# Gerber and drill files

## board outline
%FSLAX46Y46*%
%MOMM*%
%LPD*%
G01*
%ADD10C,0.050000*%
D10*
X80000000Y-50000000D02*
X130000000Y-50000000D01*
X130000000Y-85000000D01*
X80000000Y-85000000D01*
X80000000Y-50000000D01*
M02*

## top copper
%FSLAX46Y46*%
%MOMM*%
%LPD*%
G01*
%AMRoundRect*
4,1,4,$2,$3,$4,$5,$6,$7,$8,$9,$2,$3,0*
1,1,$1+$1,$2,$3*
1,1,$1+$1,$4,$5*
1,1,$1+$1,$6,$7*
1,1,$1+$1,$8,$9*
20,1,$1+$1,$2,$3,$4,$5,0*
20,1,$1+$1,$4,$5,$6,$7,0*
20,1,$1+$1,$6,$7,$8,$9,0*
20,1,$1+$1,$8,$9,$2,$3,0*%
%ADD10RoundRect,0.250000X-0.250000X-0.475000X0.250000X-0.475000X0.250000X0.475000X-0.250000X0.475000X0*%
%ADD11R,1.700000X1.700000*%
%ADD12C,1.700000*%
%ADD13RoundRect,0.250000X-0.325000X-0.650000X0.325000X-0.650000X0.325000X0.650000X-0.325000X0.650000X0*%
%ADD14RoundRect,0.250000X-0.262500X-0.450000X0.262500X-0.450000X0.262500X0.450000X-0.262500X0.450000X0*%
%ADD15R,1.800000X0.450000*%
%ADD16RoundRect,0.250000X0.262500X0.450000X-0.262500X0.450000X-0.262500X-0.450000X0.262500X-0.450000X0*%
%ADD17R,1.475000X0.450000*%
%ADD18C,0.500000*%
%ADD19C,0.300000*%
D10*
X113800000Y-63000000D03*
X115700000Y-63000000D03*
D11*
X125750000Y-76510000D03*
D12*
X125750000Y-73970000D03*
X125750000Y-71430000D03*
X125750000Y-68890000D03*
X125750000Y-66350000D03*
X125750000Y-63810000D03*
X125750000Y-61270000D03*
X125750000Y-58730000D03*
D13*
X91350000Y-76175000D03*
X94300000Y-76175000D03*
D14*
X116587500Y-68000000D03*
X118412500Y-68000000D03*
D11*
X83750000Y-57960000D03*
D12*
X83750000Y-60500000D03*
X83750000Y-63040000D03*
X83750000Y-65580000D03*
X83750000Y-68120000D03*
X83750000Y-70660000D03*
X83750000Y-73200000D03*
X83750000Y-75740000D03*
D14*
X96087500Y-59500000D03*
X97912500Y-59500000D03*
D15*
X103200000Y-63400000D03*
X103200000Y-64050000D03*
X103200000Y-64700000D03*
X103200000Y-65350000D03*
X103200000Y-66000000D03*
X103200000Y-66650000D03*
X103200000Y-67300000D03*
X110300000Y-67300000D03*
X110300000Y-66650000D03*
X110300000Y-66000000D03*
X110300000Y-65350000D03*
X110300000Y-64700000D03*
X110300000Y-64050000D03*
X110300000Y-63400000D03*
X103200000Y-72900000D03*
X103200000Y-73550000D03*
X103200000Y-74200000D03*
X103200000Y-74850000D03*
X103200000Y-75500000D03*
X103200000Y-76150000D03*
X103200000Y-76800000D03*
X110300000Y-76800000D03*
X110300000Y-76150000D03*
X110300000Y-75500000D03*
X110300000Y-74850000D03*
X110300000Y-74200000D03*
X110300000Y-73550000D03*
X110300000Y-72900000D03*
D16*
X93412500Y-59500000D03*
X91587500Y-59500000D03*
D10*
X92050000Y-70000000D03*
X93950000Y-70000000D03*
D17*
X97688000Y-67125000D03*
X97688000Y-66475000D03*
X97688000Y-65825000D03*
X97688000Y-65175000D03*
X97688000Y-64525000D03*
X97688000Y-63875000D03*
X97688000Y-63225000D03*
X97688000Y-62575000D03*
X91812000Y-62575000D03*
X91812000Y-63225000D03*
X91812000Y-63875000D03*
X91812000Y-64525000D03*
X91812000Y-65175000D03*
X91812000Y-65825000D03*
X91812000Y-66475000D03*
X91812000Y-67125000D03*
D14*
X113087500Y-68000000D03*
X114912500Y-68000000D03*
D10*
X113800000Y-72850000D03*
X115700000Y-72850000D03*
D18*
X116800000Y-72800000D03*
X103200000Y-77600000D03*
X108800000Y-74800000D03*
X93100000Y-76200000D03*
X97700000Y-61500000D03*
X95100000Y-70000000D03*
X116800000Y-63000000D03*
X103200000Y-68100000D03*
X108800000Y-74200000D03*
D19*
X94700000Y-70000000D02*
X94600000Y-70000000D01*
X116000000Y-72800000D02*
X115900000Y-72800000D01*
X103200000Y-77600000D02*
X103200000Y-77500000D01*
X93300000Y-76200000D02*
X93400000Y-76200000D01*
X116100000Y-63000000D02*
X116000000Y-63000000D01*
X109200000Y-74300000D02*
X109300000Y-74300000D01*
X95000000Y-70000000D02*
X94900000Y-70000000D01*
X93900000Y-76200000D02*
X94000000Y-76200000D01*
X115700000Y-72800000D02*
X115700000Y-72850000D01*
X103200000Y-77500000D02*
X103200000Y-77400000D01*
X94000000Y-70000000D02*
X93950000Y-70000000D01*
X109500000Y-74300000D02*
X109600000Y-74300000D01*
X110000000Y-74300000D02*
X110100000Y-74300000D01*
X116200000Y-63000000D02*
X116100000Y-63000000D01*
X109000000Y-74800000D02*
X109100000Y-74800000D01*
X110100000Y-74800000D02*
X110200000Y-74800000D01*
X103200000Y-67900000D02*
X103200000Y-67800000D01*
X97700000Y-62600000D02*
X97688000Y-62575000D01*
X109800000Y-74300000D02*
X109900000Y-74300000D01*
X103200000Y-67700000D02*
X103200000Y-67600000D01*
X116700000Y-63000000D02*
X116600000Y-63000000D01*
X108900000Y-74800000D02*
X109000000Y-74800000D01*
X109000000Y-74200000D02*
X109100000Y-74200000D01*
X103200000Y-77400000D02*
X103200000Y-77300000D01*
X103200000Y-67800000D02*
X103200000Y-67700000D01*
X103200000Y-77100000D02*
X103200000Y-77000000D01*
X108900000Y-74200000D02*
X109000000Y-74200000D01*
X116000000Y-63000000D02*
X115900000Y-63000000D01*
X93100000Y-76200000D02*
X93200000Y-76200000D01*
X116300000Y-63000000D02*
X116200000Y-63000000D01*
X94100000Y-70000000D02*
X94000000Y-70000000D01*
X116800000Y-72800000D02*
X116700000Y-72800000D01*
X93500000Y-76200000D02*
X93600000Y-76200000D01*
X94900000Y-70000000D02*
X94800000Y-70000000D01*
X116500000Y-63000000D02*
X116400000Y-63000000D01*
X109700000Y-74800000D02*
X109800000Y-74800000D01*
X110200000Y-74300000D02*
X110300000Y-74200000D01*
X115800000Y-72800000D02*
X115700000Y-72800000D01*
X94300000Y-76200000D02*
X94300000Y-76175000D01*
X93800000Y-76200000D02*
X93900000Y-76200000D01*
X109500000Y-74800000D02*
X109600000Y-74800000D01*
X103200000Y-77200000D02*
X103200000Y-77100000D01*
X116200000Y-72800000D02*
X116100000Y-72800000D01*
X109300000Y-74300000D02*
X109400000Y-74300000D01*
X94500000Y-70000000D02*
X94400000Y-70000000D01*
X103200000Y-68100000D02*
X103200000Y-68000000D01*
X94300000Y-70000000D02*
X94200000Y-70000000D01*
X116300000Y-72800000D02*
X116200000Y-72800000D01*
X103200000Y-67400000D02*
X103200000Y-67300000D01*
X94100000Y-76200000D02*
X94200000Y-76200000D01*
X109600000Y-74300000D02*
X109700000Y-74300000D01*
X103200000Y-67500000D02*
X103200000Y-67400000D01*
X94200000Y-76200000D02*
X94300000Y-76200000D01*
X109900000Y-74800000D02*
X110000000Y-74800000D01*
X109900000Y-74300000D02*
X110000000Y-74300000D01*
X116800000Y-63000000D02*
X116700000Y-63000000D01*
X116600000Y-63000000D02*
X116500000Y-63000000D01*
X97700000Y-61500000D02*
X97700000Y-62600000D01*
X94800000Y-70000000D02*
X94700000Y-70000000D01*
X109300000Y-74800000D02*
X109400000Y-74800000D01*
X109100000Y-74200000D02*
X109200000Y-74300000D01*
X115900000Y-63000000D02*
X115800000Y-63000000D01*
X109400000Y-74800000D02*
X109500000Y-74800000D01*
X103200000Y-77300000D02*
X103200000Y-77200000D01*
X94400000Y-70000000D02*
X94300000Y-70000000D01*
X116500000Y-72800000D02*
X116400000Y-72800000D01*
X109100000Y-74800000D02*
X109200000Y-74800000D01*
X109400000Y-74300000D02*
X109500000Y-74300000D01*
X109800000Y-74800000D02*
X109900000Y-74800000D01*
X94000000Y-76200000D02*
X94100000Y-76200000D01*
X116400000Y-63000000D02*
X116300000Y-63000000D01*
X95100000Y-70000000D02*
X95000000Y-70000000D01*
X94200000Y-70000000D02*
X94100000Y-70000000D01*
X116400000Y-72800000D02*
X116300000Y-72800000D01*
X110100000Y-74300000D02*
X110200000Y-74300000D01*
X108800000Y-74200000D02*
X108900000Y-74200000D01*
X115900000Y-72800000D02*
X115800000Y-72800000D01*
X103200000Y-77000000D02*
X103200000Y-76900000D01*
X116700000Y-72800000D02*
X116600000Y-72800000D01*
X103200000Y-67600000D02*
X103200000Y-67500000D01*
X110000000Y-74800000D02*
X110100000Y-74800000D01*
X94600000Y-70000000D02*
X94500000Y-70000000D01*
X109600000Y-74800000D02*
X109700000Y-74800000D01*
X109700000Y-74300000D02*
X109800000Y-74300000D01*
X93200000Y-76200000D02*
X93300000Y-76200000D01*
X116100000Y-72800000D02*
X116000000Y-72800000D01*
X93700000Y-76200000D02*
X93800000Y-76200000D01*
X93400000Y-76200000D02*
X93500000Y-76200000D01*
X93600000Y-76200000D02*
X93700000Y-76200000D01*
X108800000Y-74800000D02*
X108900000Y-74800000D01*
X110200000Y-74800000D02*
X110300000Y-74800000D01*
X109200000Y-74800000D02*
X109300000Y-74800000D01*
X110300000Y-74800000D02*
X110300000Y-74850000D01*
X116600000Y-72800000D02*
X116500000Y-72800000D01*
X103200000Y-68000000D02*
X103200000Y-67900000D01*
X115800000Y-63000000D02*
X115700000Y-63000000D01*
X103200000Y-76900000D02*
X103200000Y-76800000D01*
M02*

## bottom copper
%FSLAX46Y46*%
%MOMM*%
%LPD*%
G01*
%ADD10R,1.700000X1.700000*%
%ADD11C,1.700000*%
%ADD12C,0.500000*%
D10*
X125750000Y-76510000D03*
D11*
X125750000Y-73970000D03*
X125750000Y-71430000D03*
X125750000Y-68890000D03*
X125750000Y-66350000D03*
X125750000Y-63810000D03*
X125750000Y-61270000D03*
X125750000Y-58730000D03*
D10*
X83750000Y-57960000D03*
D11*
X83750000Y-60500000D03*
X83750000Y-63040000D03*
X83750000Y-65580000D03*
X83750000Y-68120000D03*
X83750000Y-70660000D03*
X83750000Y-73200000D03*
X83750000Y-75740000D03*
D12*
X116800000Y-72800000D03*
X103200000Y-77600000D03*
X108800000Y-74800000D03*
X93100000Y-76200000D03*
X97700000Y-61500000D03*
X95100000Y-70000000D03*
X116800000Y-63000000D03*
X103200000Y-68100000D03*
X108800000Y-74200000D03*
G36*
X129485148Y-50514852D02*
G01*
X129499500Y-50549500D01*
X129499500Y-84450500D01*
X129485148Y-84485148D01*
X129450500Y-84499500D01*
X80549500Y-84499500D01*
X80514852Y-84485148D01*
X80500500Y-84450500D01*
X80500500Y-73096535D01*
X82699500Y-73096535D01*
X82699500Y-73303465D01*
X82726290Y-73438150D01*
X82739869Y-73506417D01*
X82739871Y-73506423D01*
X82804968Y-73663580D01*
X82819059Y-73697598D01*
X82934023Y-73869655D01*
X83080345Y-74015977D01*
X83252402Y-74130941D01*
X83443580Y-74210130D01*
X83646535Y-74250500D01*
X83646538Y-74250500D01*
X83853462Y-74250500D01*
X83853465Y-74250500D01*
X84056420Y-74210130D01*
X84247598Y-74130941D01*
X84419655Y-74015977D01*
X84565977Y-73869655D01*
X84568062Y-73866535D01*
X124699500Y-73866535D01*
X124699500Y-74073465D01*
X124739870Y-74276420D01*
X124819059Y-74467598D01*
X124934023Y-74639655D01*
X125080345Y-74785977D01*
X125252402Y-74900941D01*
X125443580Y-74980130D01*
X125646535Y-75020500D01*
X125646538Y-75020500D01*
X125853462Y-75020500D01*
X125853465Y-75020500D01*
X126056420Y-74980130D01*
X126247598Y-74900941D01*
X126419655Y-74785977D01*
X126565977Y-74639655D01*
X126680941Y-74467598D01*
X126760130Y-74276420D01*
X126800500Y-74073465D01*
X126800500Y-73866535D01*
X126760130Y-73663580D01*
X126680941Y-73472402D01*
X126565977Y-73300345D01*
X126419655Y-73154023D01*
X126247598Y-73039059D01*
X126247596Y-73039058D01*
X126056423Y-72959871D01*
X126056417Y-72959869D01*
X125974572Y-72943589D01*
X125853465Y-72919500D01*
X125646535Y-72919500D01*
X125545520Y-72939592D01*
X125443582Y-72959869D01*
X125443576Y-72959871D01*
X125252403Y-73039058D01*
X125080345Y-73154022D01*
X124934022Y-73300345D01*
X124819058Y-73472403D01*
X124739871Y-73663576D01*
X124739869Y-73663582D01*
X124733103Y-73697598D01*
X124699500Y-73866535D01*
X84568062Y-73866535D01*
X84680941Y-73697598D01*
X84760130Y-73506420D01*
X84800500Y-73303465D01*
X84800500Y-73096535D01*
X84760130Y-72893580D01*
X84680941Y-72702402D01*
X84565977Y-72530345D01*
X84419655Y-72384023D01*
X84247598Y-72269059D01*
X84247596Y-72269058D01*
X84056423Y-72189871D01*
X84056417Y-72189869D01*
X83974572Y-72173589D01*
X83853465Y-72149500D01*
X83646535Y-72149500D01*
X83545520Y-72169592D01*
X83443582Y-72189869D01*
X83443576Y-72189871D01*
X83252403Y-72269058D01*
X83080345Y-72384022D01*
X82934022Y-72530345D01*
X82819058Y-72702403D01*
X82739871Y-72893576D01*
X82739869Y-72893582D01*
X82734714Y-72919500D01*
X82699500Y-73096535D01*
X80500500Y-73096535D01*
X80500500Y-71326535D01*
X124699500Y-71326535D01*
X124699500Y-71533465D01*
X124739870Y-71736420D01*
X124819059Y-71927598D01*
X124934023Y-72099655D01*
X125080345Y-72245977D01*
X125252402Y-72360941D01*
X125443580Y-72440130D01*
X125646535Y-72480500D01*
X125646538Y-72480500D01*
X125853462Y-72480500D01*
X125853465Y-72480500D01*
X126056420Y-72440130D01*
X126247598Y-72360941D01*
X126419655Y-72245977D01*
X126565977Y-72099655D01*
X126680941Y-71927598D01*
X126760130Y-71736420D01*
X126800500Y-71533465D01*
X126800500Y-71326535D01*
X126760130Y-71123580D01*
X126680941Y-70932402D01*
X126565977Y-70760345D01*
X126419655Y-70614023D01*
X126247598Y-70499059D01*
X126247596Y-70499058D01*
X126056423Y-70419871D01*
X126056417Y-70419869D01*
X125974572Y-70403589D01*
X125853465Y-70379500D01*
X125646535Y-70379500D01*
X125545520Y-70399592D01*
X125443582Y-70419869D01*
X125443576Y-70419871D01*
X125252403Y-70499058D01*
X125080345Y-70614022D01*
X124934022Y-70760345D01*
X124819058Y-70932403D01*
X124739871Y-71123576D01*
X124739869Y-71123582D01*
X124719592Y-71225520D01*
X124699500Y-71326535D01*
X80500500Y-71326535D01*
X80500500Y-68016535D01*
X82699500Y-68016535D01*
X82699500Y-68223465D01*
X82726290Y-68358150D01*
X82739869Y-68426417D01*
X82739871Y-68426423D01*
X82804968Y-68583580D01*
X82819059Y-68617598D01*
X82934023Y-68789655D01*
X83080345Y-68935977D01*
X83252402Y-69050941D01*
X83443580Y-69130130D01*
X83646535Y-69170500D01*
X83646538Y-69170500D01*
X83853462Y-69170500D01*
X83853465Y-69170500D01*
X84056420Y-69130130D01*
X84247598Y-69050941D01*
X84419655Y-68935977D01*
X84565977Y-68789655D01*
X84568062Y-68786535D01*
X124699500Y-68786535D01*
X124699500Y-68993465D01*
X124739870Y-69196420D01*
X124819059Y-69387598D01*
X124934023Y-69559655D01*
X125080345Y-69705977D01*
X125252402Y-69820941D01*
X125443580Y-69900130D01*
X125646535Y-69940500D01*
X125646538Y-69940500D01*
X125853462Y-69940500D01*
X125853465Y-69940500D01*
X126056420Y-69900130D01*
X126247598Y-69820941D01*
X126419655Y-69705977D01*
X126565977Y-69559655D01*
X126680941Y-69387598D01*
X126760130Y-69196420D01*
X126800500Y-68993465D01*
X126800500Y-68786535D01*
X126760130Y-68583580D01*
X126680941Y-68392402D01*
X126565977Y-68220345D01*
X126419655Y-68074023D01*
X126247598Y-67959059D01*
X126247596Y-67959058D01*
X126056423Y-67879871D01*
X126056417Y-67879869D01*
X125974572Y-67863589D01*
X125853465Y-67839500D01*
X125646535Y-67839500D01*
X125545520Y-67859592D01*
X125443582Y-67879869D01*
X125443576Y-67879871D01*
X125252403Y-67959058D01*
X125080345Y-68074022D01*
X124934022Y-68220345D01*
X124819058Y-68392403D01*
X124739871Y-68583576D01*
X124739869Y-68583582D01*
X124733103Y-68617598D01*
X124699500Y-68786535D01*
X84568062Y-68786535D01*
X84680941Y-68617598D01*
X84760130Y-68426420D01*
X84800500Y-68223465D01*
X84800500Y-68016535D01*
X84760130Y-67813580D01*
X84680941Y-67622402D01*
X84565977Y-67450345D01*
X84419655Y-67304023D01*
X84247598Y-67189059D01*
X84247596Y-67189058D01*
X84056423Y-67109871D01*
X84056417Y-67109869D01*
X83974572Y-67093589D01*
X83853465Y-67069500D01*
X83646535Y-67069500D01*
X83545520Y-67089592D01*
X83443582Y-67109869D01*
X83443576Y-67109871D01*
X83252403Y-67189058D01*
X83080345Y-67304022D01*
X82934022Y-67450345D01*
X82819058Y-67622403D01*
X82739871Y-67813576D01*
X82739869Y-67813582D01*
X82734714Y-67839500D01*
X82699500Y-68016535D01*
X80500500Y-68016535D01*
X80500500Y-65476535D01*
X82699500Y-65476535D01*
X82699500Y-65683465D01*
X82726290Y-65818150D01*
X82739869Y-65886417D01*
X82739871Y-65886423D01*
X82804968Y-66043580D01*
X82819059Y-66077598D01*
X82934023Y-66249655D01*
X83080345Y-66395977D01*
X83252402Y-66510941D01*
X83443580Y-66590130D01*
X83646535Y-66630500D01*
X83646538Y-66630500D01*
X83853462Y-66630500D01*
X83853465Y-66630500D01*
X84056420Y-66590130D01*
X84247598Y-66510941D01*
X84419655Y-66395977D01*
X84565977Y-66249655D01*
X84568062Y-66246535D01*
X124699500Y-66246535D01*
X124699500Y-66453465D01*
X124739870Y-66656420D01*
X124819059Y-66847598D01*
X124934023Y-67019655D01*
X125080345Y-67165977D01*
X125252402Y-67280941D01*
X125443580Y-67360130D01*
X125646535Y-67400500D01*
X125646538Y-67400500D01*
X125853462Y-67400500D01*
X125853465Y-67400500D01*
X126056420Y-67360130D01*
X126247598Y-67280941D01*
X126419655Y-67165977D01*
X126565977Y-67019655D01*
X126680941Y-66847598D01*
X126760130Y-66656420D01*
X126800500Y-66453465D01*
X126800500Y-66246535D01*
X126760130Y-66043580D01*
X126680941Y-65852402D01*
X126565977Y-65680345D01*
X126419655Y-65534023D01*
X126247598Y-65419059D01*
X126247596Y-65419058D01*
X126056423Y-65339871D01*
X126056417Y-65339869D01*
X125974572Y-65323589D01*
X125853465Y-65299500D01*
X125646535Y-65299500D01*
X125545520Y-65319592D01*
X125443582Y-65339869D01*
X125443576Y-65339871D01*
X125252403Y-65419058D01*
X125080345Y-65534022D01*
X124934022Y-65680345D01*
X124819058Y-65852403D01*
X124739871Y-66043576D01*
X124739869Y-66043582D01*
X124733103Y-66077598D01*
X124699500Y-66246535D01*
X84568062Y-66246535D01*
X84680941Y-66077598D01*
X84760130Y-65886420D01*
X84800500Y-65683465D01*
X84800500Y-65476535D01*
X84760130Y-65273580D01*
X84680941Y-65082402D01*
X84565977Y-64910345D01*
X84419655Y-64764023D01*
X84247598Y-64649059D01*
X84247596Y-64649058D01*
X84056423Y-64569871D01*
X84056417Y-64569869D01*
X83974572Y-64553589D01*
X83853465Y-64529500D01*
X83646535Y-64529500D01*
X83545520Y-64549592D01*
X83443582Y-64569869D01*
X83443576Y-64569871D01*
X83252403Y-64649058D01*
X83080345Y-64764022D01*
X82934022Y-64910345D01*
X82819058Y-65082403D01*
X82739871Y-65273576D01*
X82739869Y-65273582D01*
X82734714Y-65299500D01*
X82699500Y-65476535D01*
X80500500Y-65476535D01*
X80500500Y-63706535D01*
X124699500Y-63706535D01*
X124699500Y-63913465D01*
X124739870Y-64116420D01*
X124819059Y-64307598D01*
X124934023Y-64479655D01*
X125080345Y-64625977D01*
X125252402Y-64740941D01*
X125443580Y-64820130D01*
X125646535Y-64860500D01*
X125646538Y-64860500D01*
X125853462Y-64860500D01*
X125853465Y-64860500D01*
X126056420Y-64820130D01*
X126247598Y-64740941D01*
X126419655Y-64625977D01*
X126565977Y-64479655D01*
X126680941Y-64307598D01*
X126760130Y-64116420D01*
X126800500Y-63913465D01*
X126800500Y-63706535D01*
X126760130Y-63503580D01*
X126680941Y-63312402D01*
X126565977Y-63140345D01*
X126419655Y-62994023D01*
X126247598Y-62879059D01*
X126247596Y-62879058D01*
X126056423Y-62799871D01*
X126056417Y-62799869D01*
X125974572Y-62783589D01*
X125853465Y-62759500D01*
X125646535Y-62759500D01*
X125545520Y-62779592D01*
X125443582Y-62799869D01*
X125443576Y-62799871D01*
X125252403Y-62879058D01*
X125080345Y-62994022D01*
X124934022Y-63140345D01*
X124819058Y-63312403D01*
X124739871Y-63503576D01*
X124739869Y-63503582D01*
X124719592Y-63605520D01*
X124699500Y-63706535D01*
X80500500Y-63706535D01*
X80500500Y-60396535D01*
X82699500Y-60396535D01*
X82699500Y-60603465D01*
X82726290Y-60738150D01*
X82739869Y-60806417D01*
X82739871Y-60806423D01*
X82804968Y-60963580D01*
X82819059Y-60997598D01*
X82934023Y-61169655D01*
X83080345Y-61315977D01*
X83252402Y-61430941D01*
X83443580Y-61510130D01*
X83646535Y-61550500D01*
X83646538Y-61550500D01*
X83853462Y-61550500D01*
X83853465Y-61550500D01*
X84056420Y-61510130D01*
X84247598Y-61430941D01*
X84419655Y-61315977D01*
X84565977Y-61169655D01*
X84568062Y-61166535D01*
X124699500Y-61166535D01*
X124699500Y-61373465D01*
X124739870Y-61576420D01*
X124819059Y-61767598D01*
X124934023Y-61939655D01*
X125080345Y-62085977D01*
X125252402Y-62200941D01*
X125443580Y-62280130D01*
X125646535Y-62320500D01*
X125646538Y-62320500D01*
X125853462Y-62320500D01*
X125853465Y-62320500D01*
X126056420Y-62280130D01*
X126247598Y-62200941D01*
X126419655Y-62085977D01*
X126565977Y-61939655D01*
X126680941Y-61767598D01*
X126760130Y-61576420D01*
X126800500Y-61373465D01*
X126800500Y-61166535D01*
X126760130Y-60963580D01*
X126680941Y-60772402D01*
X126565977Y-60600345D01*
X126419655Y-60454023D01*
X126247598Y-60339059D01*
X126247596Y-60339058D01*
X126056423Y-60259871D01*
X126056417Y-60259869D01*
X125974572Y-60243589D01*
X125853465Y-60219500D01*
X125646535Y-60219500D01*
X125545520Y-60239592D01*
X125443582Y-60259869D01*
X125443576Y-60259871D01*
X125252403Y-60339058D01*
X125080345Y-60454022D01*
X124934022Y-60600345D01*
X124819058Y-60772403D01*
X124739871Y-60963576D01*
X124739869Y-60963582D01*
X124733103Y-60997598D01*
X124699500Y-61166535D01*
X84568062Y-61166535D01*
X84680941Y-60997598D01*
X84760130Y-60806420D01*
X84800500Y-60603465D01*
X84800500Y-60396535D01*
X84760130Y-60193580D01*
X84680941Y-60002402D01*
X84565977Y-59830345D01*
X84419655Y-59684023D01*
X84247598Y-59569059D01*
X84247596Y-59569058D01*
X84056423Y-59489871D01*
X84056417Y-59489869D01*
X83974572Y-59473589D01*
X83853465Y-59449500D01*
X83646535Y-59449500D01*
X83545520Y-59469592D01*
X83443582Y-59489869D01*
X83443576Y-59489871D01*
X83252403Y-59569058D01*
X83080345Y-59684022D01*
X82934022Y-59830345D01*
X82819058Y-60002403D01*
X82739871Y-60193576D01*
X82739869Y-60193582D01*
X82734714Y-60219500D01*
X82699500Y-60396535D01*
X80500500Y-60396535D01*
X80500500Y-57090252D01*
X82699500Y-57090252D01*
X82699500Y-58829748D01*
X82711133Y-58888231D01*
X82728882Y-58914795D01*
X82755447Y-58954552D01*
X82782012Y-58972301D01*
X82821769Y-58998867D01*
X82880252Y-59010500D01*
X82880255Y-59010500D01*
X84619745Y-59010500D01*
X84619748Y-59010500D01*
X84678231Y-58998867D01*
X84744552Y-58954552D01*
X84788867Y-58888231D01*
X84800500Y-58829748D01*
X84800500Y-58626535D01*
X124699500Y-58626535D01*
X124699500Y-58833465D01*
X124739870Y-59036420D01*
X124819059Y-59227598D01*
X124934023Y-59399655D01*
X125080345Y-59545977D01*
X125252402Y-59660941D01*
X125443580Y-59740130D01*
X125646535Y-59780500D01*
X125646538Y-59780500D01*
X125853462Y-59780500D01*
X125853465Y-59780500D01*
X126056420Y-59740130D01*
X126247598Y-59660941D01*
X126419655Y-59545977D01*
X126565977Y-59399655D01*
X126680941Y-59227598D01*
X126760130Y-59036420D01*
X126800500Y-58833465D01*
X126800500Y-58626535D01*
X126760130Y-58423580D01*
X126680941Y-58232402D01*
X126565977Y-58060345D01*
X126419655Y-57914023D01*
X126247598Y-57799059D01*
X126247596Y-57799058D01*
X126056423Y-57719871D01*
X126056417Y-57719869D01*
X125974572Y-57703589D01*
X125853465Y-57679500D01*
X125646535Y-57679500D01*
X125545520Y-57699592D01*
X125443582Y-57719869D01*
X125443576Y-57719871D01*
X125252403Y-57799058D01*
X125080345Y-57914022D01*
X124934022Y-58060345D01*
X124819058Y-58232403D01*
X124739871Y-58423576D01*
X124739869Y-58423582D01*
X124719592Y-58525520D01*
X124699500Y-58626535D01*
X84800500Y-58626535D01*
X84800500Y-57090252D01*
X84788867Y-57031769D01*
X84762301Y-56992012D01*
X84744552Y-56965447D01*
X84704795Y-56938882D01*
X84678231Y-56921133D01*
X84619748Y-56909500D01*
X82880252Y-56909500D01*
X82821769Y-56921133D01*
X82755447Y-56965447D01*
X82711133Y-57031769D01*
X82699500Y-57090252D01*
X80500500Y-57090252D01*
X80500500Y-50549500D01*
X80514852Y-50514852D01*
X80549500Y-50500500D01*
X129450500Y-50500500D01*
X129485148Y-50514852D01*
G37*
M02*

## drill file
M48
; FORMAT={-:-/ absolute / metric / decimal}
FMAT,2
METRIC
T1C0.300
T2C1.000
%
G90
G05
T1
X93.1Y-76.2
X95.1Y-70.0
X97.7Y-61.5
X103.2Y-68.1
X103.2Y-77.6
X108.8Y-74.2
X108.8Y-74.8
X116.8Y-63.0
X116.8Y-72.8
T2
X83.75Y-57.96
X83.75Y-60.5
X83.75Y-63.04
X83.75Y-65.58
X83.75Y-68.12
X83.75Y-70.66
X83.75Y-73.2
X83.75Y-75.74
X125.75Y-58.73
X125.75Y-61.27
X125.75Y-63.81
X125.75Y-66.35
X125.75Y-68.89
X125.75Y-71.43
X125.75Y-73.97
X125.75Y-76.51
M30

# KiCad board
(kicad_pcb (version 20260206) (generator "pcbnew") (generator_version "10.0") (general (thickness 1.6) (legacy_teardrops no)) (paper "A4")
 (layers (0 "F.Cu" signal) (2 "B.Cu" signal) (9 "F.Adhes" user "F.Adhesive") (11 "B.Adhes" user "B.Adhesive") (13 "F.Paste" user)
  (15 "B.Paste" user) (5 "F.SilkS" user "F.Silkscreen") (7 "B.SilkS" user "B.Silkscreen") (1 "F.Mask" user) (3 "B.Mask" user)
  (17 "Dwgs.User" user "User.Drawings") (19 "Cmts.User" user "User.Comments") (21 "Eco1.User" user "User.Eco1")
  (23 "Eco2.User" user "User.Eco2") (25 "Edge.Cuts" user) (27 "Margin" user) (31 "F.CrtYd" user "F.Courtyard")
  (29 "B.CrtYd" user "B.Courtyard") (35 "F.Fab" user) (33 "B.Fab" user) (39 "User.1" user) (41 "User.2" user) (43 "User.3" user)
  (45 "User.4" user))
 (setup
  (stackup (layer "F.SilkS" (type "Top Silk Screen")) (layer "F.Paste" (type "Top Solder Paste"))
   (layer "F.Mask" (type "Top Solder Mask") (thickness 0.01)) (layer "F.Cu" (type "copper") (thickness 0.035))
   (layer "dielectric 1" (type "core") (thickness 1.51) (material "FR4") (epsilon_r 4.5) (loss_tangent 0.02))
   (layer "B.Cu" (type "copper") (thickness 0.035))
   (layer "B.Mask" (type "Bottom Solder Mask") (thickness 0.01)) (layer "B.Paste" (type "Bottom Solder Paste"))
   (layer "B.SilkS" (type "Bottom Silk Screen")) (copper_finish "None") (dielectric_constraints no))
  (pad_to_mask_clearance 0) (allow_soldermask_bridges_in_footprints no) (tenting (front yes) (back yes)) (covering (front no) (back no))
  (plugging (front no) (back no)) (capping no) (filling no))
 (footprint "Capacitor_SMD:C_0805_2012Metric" (layer "F.Cu") (at 114.75 63)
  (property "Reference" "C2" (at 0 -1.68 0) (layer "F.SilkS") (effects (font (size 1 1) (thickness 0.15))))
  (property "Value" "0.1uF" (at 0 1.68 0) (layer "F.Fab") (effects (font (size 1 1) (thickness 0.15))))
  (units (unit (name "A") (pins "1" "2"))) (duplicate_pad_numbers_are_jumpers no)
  (pad "1" smd roundrect (at -0.95 0) (size 1 1.45) (layers "F.Cu" "F.Mask" "F.Paste") (roundrect_rratio 0.25) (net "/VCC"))
  (pad "2" smd roundrect (at 0.95 0) (size 1 1.45) (layers "F.Cu" "F.Mask" "F.Paste") (roundrect_rratio 0.25) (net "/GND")))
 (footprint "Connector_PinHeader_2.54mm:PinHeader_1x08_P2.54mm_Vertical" (layer "F.Cu") (at 125.75 76.51 180)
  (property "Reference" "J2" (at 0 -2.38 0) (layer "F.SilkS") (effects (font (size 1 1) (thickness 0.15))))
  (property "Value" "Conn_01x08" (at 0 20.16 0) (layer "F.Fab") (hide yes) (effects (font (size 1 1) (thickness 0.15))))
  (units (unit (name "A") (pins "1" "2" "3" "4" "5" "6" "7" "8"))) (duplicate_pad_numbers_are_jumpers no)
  (pad "1" thru_hole rect (at 0 0 180) (size 1.7 1.7) (drill 1) (layers "*.Cu" "*.Mask") (remove_unused_layers no) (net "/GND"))
  (pad "2" thru_hole circle (at 0 2.54 180) (size 1.7 1.7) (drill 1) (layers "*.Cu" "*.Mask") (remove_unused_layers no) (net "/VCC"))
  (pad "3" thru_hole circle (at 0 5.08 180) (size 1.7 1.7) (drill 1) (layers "*.Cu" "*.Mask") (remove_unused_layers no) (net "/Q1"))
  (pad "4" thru_hole circle (at 0 7.62 180) (size 1.7 1.7) (drill 1) (layers "*.Cu" "*.Mask") (remove_unused_layers no) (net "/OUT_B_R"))
  (pad "5" thru_hole circle (at 0 10.16 180) (size 1.7 1.7) (drill 1) (layers "*.Cu" "*.Mask") (remove_unused_layers no) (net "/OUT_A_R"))
  (pad "6" thru_hole circle (at 0 12.7 180) (size 1.7 1.7) (drill 1) (layers "*.Cu" "*.Mask") (remove_unused_layers no) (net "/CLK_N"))
  (pad "7" thru_hole circle (at 0 15.24 180) (size 1.7 1.7) (drill 1) (layers "*.Cu" "*.Mask") (remove_unused_layers no) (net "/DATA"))
  (pad "8" thru_hole circle (at 0 17.78 180) (size 1.7 1.7) (drill 1) (layers "*.Cu" "*.Mask") (remove_unused_layers no) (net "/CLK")))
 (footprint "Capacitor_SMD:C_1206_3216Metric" (layer "F.Cu") (at 92.825 76.175)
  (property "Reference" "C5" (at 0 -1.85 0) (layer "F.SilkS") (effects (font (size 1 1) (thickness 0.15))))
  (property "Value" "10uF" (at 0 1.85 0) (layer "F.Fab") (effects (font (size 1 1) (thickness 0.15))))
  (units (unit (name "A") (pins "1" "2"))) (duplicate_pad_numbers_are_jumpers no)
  (pad "1" smd roundrect (at -1.475 0) (size 1.15 1.8) (layers "F.Cu" "F.Mask" "F.Paste") (roundrect_rratio 0.217391) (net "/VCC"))
  (pad "2" smd roundrect (at 1.475 0) (size 1.15 1.8) (layers "F.Cu" "F.Mask" "F.Paste") (roundrect_rratio 0.217391) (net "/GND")))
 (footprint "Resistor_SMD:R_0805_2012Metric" (layer "F.Cu") (at 117.5 68)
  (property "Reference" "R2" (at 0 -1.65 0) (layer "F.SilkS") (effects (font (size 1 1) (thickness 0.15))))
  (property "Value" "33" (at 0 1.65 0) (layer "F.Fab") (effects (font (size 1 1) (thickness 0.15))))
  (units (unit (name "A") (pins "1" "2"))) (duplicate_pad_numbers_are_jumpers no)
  (pad "1" smd roundrect (at -0.9125 0) (size 1.025 1.4) (layers "F.Cu" "F.Mask" "F.Paste") (roundrect_rratio 0.243902) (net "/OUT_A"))
  (pad "2" smd roundrect (at 0.9125 0) (size 1.025 1.4) (layers "F.Cu" "F.Mask" "F.Paste") (roundrect_rratio 0.243902) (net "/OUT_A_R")))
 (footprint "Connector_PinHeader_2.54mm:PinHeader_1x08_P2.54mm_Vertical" (layer "F.Cu") (at 83.75 57.96)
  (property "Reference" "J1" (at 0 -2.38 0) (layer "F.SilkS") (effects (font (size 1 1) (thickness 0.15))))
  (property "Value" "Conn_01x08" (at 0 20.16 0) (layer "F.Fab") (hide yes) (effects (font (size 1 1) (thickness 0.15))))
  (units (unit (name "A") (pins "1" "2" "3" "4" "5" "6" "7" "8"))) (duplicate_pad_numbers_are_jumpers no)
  (pad "1" thru_hole rect (at 0 0) (size 1.7 1.7) (drill 1) (layers "*.Cu" "*.Mask") (remove_unused_layers no) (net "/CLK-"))
  (pad "2" thru_hole circle (at 0 2.54) (size 1.7 1.7) (drill 1) (layers "*.Cu" "*.Mask") (remove_unused_layers no) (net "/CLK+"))
  (pad "3" thru_hole circle (at 0 5.08) (size 1.7 1.7) (drill 1) (layers "*.Cu" "*.Mask") (remove_unused_layers no) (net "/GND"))
  (pad "4" thru_hole circle (at 0 7.62) (size 1.7 1.7) (drill 1) (layers "*.Cu" "*.Mask") (remove_unused_layers no) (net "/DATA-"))
  (pad "5" thru_hole circle (at 0 10.16) (size 1.7 1.7) (drill 1) (layers "*.Cu" "*.Mask") (remove_unused_layers no) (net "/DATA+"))
  (pad "6" thru_hole circle (at 0 12.7) (size 1.7 1.7) (drill 1) (layers "*.Cu" "*.Mask") (remove_unused_layers no) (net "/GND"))
  (pad "7" thru_hole circle (at 0 15.24) (size 1.7 1.7) (drill 1) (layers "*.Cu" "*.Mask") (remove_unused_layers no) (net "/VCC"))
  (pad "8" thru_hole circle (at 0 17.78) (size 1.7 1.7) (drill 1) (layers "*.Cu" "*.Mask") (remove_unused_layers no) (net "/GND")))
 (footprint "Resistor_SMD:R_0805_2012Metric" (layer "F.Cu") (at 97 59.5)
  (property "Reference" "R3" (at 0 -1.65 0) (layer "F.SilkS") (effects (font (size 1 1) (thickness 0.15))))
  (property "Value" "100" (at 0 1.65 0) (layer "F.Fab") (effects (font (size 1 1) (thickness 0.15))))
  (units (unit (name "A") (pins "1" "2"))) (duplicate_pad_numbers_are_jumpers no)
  (pad "1" smd roundrect (at -0.9125 0) (size 1.025 1.4) (layers "F.Cu" "F.Mask" "F.Paste") (roundrect_rratio 0.243902) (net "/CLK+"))
  (pad "2" smd roundrect (at 0.9125 0) (size 1.025 1.4) (layers "F.Cu" "F.Mask" "F.Paste") (roundrect_rratio 0.243902) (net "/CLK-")))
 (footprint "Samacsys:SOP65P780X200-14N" (layer "F.Cu") (at 106.75 65.35)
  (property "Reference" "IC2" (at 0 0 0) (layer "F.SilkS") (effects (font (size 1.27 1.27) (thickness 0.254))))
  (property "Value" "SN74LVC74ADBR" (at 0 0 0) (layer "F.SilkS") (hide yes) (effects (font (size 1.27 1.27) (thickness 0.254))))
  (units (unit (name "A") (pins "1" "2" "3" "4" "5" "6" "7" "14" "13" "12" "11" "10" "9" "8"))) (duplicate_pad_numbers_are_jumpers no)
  (pad "1" smd rect (at -3.55 -1.95 90) (size 0.45 1.8) (layers "F.Cu" "F.Mask" "F.Paste") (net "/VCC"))
  (pad "2" smd rect (at -3.55 -1.3 90) (size 0.45 1.8) (layers "F.Cu" "F.Mask" "F.Paste") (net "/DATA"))
  (pad "3" smd rect (at -3.55 -0.65 90) (size 0.45 1.8) (layers "F.Cu" "F.Mask" "F.Paste") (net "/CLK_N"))
  (pad "4" smd rect (at -3.55 0 90) (size 0.45 1.8) (layers "F.Cu" "F.Mask" "F.Paste") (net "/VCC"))
  (pad "5" smd rect (at -3.55 0.65 90) (size 0.45 1.8) (layers "F.Cu" "F.Mask" "F.Paste") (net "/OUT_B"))
  (pad "6" smd rect (at -3.55 1.3 90) (size 0.45 1.8) (layers "F.Cu" "F.Mask" "F.Paste") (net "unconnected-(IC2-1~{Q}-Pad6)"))
  (pad "7" smd rect (at -3.55 1.95 90) (size 0.45 1.8) (layers "F.Cu" "F.Mask" "F.Paste") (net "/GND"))
  (pad "8" smd rect (at 3.55 1.95 90) (size 0.45 1.8) (layers "F.Cu" "F.Mask" "F.Paste") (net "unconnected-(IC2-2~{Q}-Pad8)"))
  (pad "9" smd rect (at 3.55 1.3 90) (size 0.45 1.8) (layers "F.Cu" "F.Mask" "F.Paste") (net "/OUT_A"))
  (pad "10" smd rect (at 3.55 0.65 90) (size 0.45 1.8) (layers "F.Cu" "F.Mask" "F.Paste") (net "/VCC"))
  (pad "11" smd rect (at 3.55 0 90) (size 0.45 1.8) (layers "F.Cu" "F.Mask" "F.Paste") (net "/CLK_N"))
  (pad "12" smd rect (at 3.55 -0.65 90) (size 0.45 1.8) (layers "F.Cu" "F.Mask" "F.Paste") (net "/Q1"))
  (pad "13" smd rect (at 3.55 -1.3 90) (size 0.45 1.8) (layers "F.Cu" "F.Mask" "F.Paste") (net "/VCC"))
  (pad "14" smd rect (at 3.55 -1.95 90) (size 0.45 1.8) (layers "F.Cu" "F.Mask" "F.Paste") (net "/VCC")))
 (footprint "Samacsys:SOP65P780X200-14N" (layer "F.Cu") (at 106.75 74.85)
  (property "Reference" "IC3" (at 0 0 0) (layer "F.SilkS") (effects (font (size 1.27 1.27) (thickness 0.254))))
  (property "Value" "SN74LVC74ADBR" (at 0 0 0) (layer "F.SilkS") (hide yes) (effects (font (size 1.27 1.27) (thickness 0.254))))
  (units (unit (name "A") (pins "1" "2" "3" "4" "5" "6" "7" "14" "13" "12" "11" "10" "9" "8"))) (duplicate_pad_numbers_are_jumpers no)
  (pad "1" smd rect (at -3.55 -1.95 90) (size 0.45 1.8) (layers "F.Cu" "F.Mask" "F.Paste") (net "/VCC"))
  (pad "2" smd rect (at -3.55 -1.3 90) (size 0.45 1.8) (layers "F.Cu" "F.Mask" "F.Paste") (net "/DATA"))
  (pad "3" smd rect (at -3.55 -0.65 90) (size 0.45 1.8) (layers "F.Cu" "F.Mask" "F.Paste") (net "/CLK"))
  (pad "4" smd rect (at -3.55 0 90) (size 0.45 1.8) (layers "F.Cu" "F.Mask" "F.Paste") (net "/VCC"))
  (pad "5" smd rect (at -3.55 0.65 90) (size 0.45 1.8) (layers "F.Cu" "F.Mask" "F.Paste") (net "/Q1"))
  (pad "6" smd rect (at -3.55 1.3 90) (size 0.45 1.8) (layers "F.Cu" "F.Mask" "F.Paste") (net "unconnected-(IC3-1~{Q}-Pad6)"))
  (pad "7" smd rect (at -3.55 1.95 90) (size 0.45 1.8) (layers "F.Cu" "F.Mask" "F.Paste") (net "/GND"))
  (pad "8" smd rect (at 3.55 1.95 90) (size 0.45 1.8) (layers "F.Cu" "F.Mask" "F.Paste") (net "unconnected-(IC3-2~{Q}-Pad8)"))
  (pad "9" smd rect (at 3.55 1.3 90) (size 0.45 1.8) (layers "F.Cu" "F.Mask" "F.Paste") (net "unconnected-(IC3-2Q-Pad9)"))
  (pad "10" smd rect (at 3.55 0.65 90) (size 0.45 1.8) (layers "F.Cu" "F.Mask" "F.Paste") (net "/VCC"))
  (pad "11" smd rect (at 3.55 0 90) (size 0.45 1.8) (layers "F.Cu" "F.Mask" "F.Paste") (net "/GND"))
  (pad "12" smd rect (at 3.55 -0.65 90) (size 0.45 1.8) (layers "F.Cu" "F.Mask" "F.Paste") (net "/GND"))
  (pad "13" smd rect (at 3.55 -1.3 90) (size 0.45 1.8) (layers "F.Cu" "F.Mask" "F.Paste") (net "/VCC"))
  (pad "14" smd rect (at 3.55 -1.95 90) (size 0.45 1.8) (layers "F.Cu" "F.Mask" "F.Paste") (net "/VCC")))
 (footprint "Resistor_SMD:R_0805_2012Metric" (layer "F.Cu") (at 92.5 59.5 180)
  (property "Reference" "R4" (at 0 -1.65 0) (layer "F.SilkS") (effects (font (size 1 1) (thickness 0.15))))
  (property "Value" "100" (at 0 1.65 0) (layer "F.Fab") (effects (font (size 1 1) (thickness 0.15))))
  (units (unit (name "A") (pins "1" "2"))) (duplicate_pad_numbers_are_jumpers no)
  (pad "1" smd roundrect (at -0.9125 0 180) (size 1.025 1.4) (layers "F.Cu" "F.Mask" "F.Paste") (roundrect_rratio 0.243902) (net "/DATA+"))
  (pad "2" smd roundrect (at 0.9125 0 180) (size 1.025 1.4) (layers "F.Cu" "F.Mask" "F.Paste") (roundrect_rratio 0.243902) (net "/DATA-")))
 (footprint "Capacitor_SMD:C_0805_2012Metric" (layer "F.Cu") (at 93 70)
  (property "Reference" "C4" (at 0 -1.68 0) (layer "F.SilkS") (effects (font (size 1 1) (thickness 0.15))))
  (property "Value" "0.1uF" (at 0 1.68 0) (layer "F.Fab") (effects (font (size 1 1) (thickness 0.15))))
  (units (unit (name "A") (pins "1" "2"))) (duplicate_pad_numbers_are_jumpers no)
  (pad "1" smd roundrect (at -0.95 0) (size 1 1.45) (layers "F.Cu" "F.Mask" "F.Paste") (roundrect_rratio 0.25) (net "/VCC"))
  (pad "2" smd roundrect (at 0.95 0) (size 1 1.45) (layers "F.Cu" "F.Mask" "F.Paste") (roundrect_rratio 0.25) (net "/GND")))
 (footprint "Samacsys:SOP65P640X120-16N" (layer "F.Cu") (at 94.75 64.85 180)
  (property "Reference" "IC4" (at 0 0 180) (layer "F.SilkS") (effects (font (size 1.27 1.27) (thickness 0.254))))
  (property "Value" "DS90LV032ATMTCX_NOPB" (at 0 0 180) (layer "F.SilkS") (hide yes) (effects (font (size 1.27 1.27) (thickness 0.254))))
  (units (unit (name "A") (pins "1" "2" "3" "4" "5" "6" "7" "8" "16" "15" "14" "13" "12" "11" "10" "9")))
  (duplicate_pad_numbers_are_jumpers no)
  (pad "1" smd rect (at -2.938 -2.275 270) (size 0.45 1.475) (layers "F.Cu" "F.Mask" "F.Paste") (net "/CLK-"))
  (pad "2" smd rect (at -2.938 -1.625 270) (size 0.45 1.475) (layers "F.Cu" "F.Mask" "F.Paste") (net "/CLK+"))
  (pad "3" smd rect (at -2.938 -0.975 270) (size 0.45 1.475) (layers "F.Cu" "F.Mask" "F.Paste") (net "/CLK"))
  (pad "4" smd rect (at -2.938 -0.325 270) (size 0.45 1.475) (layers "F.Cu" "F.Mask" "F.Paste") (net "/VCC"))
  (pad "5" smd rect (at -2.938 0.325 270) (size 0.45 1.475) (layers "F.Cu" "F.Mask" "F.Paste") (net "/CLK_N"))
  (pad "6" smd rect (at -2.938 0.975 270) (size 0.45 1.475) (layers "F.Cu" "F.Mask" "F.Paste") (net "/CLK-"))
  (pad "7" smd rect (at -2.938 1.625 270) (size 0.45 1.475) (layers "F.Cu" "F.Mask" "F.Paste") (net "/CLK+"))
  (pad "8" smd rect (at -2.938 2.275 270) (size 0.45 1.475) (layers "F.Cu" "F.Mask" "F.Paste") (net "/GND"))
  (pad "9" smd rect (at 2.938 2.275 270) (size 0.45 1.475) (layers "F.Cu" "F.Mask" "F.Paste") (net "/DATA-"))
  (pad "10" smd rect (at 2.938 1.625 270) (size 0.45 1.475) (layers "F.Cu" "F.Mask" "F.Paste") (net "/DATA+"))
  (pad "11" smd rect (at 2.938 0.975 270) (size 0.45 1.475) (layers "F.Cu" "F.Mask" "F.Paste") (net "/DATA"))
  (pad "12" smd rect (at 2.938 0.325 270) (size 0.45 1.475) (layers "F.Cu" "F.Mask" "F.Paste") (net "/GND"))
  (pad "13" smd rect (at 2.938 -0.325 270) (size 0.45 1.475) (layers "F.Cu" "F.Mask" "F.Paste") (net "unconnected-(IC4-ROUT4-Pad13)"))
  (pad "14" smd rect (at 2.938 -0.975 270) (size 0.45 1.475) (layers "F.Cu" "F.Mask" "F.Paste") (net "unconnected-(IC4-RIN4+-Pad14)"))
  (pad "15" smd rect (at 2.938 -1.625 270) (size 0.45 1.475) (layers "F.Cu" "F.Mask" "F.Paste") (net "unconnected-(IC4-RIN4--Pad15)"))
  (pad "16" smd rect (at 2.938 -2.275 270) (size 0.45 1.475) (layers "F.Cu" "F.Mask" "F.Paste") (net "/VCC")))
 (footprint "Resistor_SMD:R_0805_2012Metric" (layer "F.Cu") (at 114 68)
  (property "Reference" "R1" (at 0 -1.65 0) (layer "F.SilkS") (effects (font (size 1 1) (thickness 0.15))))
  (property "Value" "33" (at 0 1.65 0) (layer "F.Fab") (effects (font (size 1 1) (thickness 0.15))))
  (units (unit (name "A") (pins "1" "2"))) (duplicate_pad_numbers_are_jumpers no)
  (pad "1" smd roundrect (at -0.9125 0) (size 1.025 1.4) (layers "F.Cu" "F.Mask" "F.Paste") (roundrect_rratio 0.243902) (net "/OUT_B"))
  (pad "2" smd roundrect (at 0.9125 0) (size 1.025 1.4) (layers "F.Cu" "F.Mask" "F.Paste") (roundrect_rratio 0.243902) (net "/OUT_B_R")))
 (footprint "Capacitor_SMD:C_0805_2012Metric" (layer "F.Cu") (at 114.75 72.85)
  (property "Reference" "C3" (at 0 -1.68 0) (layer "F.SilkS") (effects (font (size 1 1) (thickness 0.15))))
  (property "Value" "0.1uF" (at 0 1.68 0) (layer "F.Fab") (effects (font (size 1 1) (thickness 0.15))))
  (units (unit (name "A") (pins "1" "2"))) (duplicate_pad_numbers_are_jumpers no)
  (pad "1" smd roundrect (at -0.95 0) (size 1 1.45) (layers "F.Cu" "F.Mask" "F.Paste") (roundrect_rratio 0.25) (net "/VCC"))
  (pad "2" smd roundrect (at 0.95 0) (size 1 1.45) (layers "F.Cu" "F.Mask" "F.Paste") (roundrect_rratio 0.25) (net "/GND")))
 (gr_poly (pts (xy 80 50) (xy 130 50) (xy 130 85) (xy 80 85)) (stroke (width 0.05) (type solid)) (fill no) (layer "Edge.Cuts"))
 (segment (start 94.7 70) (end 94.6 70) (width 0.3) (layer "F.Cu") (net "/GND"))
 (segment (start 116 72.8) (end 115.9 72.8) (width 0.3) (layer "F.Cu") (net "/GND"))
 (segment (start 103.2 77.6) (end 103.2 77.5) (width 0.3) (layer "F.Cu") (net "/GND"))
 (segment (start 93.3 76.2) (end 93.4 76.2) (width 0.3) (layer "F.Cu") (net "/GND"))
 (segment (start 116.1 63) (end 116 63) (width 0.3) (layer "F.Cu") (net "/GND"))
 (segment (start 109.2 74.3) (end 109.3 74.3) (width 0.3) (layer "F.Cu") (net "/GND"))
 (segment (start 95 70) (end 94.9 70) (width 0.3) (layer "F.Cu") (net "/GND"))
 (segment (start 93.9 76.2) (end 94 76.2) (width 0.3) (layer "F.Cu") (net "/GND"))
 (segment (start 115.7 72.8) (end 115.7 72.85) (width 0.3) (layer "F.Cu") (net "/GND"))
 (segment (start 103.2 77.5) (end 103.2 77.4) (width 0.3) (layer "F.Cu") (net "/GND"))
 (segment (start 94 70) (end 93.95 70) (width 0.3) (layer "F.Cu") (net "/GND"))
 (segment (start 109.5 74.3) (end 109.6 74.3) (width 0.3) (layer "F.Cu") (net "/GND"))
 (segment (start 110 74.3) (end 110.1 74.3) (width 0.3) (layer "F.Cu") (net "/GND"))
 (segment (start 116.2 63) (end 116.1 63) (width 0.3) (layer "F.Cu") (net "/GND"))
 (segment (start 109 74.8) (end 109.1 74.8) (width 0.3) (layer "F.Cu") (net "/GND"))
 (segment (start 110.1 74.8) (end 110.2 74.8) (width 0.3) (layer "F.Cu") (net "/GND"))
 (segment (start 103.2 67.9) (end 103.2 67.8) (width 0.3) (layer "F.Cu") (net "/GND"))
 (segment (start 97.7 62.6) (end 97.688 62.575) (width 0.3) (layer "F.Cu") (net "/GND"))
 (segment (start 109.8 74.3) (end 109.9 74.3) (width 0.3) (layer "F.Cu") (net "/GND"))
 (segment (start 103.2 67.7) (end 103.2 67.6) (width 0.3) (layer "F.Cu") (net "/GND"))
 (segment (start 116.7 63) (end 116.6 63) (width 0.3) (layer "F.Cu") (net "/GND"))
 (segment (start 108.9 74.8) (end 109 74.8) (width 0.3) (layer "F.Cu") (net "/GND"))
 (segment (start 109 74.2) (end 109.1 74.2) (width 0.3) (layer "F.Cu") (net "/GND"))
 (segment (start 103.2 77.4) (end 103.2 77.3) (width 0.3) (layer "F.Cu") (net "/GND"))
 (segment (start 103.2 67.8) (end 103.2 67.7) (width 0.3) (layer "F.Cu") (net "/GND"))
 (segment (start 103.2 77.1) (end 103.2 77) (width 0.3) (layer "F.Cu") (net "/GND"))
 (segment (start 108.9 74.2) (end 109 74.2) (width 0.3) (layer "F.Cu") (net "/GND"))
 (segment (start 116 63) (end 115.9 63) (width 0.3) (layer "F.Cu") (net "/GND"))
 (segment (start 93.1 76.2) (end 93.2 76.2) (width 0.3) (layer "F.Cu") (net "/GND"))
 (segment (start 116.3 63) (end 116.2 63) (width 0.3) (layer "F.Cu") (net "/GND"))
 (segment (start 94.1 70) (end 94 70) (width 0.3) (layer "F.Cu") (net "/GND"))
 (segment (start 116.8 72.8) (end 116.7 72.8) (width 0.3) (layer "F.Cu") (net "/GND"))
 (segment (start 93.5 76.2) (end 93.6 76.2) (width 0.3) (layer "F.Cu") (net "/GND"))
 (segment (start 94.9 70) (end 94.8 70) (width 0.3) (layer "F.Cu") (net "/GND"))
 (segment (start 116.5 63) (end 116.4 63) (width 0.3) (layer "F.Cu") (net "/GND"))
 (segment (start 109.7 74.8) (end 109.8 74.8) (width 0.3) (layer "F.Cu") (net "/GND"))
 (segment (start 110.2 74.3) (end 110.3 74.2) (width 0.3) (layer "F.Cu") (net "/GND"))
 (segment (start 115.8 72.8) (end 115.7 72.8) (width 0.3) (layer "F.Cu") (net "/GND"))
 (segment (start 94.3 76.2) (end 94.3 76.175) (width 0.3) (layer "F.Cu") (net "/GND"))
 (segment (start 93.8 76.2) (end 93.9 76.2) (width 0.3) (layer "F.Cu") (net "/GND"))
 (segment (start 109.5 74.8) (end 109.6 74.8) (width 0.3) (layer "F.Cu") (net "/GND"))
 (segment (start 103.2 77.2) (end 103.2 77.1) (width 0.3) (layer "F.Cu") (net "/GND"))
 (segment (start 116.2 72.8) (end 116.1 72.8) (width 0.3) (layer "F.Cu") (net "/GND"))
 (segment (start 109.3 74.3) (end 109.4 74.3) (width 0.3) (layer "F.Cu") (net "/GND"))
 (segment (start 94.5 70) (end 94.4 70) (width 0.3) (layer "F.Cu") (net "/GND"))
 (segment (start 103.2 68.1) (end 103.2 68) (width 0.3) (layer "F.Cu") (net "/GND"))
 (segment (start 94.3 70) (end 94.2 70) (width 0.3) (layer "F.Cu") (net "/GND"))
 (segment (start 116.3 72.8) (end 116.2 72.8) (width 0.3) (layer "F.Cu") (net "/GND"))
 (segment (start 103.2 67.4) (end 103.2 67.3) (width 0.3) (layer "F.Cu") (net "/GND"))
 (segment (start 94.1 76.2) (end 94.2 76.2) (width 0.3) (layer "F.Cu") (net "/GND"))
 (segment (start 109.6 74.3) (end 109.7 74.3) (width 0.3) (layer "F.Cu") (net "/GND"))
 (segment (start 103.2 67.5) (end 103.2 67.4) (width 0.3) (layer "F.Cu") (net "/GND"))
 (segment (start 94.2 76.2) (end 94.3 76.2) (width 0.3) (layer "F.Cu") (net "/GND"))
 (segment (start 109.9 74.8) (end 110 74.8) (width 0.3) (layer "F.Cu") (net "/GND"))
 (segment (start 109.9 74.3) (end 110 74.3) (width 0.3) (layer "F.Cu") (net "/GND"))
 (segment (start 116.8 63) (end 116.7 63) (width 0.3) (layer "F.Cu") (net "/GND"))
 (segment (start 116.6 63) (end 116.5 63) (width 0.3) (layer "F.Cu") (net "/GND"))
 (segment (start 97.7 61.5) (end 97.7 62.6) (width 0.3) (layer "F.Cu") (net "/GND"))
 (segment (start 94.8 70) (end 94.7 70) (width 0.3) (layer "F.Cu") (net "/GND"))
 (segment (start 109.3 74.8) (end 109.4 74.8) (width 0.3) (layer "F.Cu") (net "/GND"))
 (segment (start 109.1 74.2) (end 109.2 74.3) (width 0.3) (layer "F.Cu") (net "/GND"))
 (segment (start 115.9 63) (end 115.8 63) (width 0.3) (layer "F.Cu") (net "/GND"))
 (segment (start 109.4 74.8) (end 109.5 74.8) (width 0.3) (layer "F.Cu") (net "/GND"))
 (segment (start 103.2 77.3) (end 103.2 77.2) (width 0.3) (layer "F.Cu") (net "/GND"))
 (segment (start 94.4 70) (end 94.3 70) (width 0.3) (layer "F.Cu") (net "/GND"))
 (segment (start 116.5 72.8) (end 116.4 72.8) (width 0.3) (layer "F.Cu") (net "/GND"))
 (segment (start 109.1 74.8) (end 109.2 74.8) (width 0.3) (layer "F.Cu") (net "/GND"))
 (segment (start 109.4 74.3) (end 109.5 74.3) (width 0.3) (layer "F.Cu") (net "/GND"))
 (segment (start 109.8 74.8) (end 109.9 74.8) (width 0.3) (layer "F.Cu") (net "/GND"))
 (segment (start 94 76.2) (end 94.1 76.2) (width 0.3) (layer "F.Cu") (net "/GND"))
 (segment (start 116.4 63) (end 116.3 63) (width 0.3) (layer "F.Cu") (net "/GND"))
 (segment (start 95.1 70) (end 95 70) (width 0.3) (layer "F.Cu") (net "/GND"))
 (segment (start 94.2 70) (end 94.1 70) (width 0.3) (layer "F.Cu") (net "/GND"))
 (segment (start 116.4 72.8) (end 116.3 72.8) (width 0.3) (layer "F.Cu") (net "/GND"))
 (segment (start 110.1 74.3) (end 110.2 74.3) (width 0.3) (layer "F.Cu") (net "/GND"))
 (segment (start 108.8 74.2) (end 108.9 74.2) (width 0.3) (layer "F.Cu") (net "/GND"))
 (segment (start 115.9 72.8) (end 115.8 72.8) (width 0.3) (layer "F.Cu") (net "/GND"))
 (segment (start 103.2 77) (end 103.2 76.9) (width 0.3) (layer "F.Cu") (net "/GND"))
 (segment (start 116.7 72.8) (end 116.6 72.8) (width 0.3) (layer "F.Cu") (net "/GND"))
 (segment (start 103.2 67.6) (end 103.2 67.5) (width 0.3) (layer "F.Cu") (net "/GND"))
 (segment (start 110 74.8) (end 110.1 74.8) (width 0.3) (layer "F.Cu") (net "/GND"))
 (segment (start 94.6 70) (end 94.5 70) (width 0.3) (layer "F.Cu") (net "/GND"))
 (segment (start 109.6 74.8) (end 109.7 74.8) (width 0.3) (layer "F.Cu") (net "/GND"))
 (segment (start 109.7 74.3) (end 109.8 74.3) (width 0.3) (layer "F.Cu") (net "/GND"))
 (segment (start 93.2 76.2) (end 93.3 76.2) (width 0.3) (layer "F.Cu") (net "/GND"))
 (segment (start 116.1 72.8) (end 116 72.8) (width 0.3) (layer "F.Cu") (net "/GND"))
 (segment (start 93.7 76.2) (end 93.8 76.2) (width 0.3) (layer "F.Cu") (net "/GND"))
 (segment (start 93.4 76.2) (end 93.5 76.2) (width 0.3) (layer "F.Cu") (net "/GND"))
 (segment (start 93.6 76.2) (end 93.7 76.2) (width 0.3) (layer "F.Cu") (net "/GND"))
 (segment (start 108.8 74.8) (end 108.9 74.8) (width 0.3) (layer "F.Cu") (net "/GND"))
 (segment (start 110.2 74.8) (end 110.3 74.8) (width 0.3) (layer "F.Cu") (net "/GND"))
 (segment (start 109.2 74.8) (end 109.3 74.8) (width 0.3) (layer "F.Cu") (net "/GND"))
 (segment (start 110.3 74.8) (end 110.3 74.85) (width 0.3) (layer "F.Cu") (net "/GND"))
 (segment (start 116.6 72.8) (end 116.5 72.8) (width 0.3) (layer "F.Cu") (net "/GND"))
 (segment (start 103.2 68) (end 103.2 67.9) (width 0.3) (layer "F.Cu") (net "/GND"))
 (segment (start 115.8 63) (end 115.7 63) (width 0.3) (layer "F.Cu") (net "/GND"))
 (segment (start 103.2 76.9) (end 103.2 76.8) (width 0.3) (layer "F.Cu") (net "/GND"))
 (via (at 116.8 72.8) (size 0.5) (drill 0.3) (layers "F.Cu" "B.Cu") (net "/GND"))
 (via (at 103.2 77.6) (size 0.5) (drill 0.3) (layers "F.Cu" "B.Cu") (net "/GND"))
 (via (at 108.8 74.8) (size 0.5) (drill 0.3) (layers "F.Cu" "B.Cu") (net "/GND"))
 (via (at 93.1 76.2) (size 0.5) (drill 0.3) (layers "F.Cu" "B.Cu") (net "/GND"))
 (via (at 97.7 61.5) (size 0.5) (drill 0.3) (layers "F.Cu" "B.Cu") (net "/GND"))
 (via (at 95.1 70) (size 0.5) (drill 0.3) (layers "F.Cu" "B.Cu") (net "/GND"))
 (via (at 116.8 63) (size 0.5) (drill 0.3) (layers "F.Cu" "B.Cu") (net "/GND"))
 (via (at 103.2 68.1) (size 0.5) (drill 0.3) (layers "F.Cu" "B.Cu") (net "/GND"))
 (via (at 108.8 74.2) (size 0.5) (drill 0.3) (layers "F.Cu" "B.Cu") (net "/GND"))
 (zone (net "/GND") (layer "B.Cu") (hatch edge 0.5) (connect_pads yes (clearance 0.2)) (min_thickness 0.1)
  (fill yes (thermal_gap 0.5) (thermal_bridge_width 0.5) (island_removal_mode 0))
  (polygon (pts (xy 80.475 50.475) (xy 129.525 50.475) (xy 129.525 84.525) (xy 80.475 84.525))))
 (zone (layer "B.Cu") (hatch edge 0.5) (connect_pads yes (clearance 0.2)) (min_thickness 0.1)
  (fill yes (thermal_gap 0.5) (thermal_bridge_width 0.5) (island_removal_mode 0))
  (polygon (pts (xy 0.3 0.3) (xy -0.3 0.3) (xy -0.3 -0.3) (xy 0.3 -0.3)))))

